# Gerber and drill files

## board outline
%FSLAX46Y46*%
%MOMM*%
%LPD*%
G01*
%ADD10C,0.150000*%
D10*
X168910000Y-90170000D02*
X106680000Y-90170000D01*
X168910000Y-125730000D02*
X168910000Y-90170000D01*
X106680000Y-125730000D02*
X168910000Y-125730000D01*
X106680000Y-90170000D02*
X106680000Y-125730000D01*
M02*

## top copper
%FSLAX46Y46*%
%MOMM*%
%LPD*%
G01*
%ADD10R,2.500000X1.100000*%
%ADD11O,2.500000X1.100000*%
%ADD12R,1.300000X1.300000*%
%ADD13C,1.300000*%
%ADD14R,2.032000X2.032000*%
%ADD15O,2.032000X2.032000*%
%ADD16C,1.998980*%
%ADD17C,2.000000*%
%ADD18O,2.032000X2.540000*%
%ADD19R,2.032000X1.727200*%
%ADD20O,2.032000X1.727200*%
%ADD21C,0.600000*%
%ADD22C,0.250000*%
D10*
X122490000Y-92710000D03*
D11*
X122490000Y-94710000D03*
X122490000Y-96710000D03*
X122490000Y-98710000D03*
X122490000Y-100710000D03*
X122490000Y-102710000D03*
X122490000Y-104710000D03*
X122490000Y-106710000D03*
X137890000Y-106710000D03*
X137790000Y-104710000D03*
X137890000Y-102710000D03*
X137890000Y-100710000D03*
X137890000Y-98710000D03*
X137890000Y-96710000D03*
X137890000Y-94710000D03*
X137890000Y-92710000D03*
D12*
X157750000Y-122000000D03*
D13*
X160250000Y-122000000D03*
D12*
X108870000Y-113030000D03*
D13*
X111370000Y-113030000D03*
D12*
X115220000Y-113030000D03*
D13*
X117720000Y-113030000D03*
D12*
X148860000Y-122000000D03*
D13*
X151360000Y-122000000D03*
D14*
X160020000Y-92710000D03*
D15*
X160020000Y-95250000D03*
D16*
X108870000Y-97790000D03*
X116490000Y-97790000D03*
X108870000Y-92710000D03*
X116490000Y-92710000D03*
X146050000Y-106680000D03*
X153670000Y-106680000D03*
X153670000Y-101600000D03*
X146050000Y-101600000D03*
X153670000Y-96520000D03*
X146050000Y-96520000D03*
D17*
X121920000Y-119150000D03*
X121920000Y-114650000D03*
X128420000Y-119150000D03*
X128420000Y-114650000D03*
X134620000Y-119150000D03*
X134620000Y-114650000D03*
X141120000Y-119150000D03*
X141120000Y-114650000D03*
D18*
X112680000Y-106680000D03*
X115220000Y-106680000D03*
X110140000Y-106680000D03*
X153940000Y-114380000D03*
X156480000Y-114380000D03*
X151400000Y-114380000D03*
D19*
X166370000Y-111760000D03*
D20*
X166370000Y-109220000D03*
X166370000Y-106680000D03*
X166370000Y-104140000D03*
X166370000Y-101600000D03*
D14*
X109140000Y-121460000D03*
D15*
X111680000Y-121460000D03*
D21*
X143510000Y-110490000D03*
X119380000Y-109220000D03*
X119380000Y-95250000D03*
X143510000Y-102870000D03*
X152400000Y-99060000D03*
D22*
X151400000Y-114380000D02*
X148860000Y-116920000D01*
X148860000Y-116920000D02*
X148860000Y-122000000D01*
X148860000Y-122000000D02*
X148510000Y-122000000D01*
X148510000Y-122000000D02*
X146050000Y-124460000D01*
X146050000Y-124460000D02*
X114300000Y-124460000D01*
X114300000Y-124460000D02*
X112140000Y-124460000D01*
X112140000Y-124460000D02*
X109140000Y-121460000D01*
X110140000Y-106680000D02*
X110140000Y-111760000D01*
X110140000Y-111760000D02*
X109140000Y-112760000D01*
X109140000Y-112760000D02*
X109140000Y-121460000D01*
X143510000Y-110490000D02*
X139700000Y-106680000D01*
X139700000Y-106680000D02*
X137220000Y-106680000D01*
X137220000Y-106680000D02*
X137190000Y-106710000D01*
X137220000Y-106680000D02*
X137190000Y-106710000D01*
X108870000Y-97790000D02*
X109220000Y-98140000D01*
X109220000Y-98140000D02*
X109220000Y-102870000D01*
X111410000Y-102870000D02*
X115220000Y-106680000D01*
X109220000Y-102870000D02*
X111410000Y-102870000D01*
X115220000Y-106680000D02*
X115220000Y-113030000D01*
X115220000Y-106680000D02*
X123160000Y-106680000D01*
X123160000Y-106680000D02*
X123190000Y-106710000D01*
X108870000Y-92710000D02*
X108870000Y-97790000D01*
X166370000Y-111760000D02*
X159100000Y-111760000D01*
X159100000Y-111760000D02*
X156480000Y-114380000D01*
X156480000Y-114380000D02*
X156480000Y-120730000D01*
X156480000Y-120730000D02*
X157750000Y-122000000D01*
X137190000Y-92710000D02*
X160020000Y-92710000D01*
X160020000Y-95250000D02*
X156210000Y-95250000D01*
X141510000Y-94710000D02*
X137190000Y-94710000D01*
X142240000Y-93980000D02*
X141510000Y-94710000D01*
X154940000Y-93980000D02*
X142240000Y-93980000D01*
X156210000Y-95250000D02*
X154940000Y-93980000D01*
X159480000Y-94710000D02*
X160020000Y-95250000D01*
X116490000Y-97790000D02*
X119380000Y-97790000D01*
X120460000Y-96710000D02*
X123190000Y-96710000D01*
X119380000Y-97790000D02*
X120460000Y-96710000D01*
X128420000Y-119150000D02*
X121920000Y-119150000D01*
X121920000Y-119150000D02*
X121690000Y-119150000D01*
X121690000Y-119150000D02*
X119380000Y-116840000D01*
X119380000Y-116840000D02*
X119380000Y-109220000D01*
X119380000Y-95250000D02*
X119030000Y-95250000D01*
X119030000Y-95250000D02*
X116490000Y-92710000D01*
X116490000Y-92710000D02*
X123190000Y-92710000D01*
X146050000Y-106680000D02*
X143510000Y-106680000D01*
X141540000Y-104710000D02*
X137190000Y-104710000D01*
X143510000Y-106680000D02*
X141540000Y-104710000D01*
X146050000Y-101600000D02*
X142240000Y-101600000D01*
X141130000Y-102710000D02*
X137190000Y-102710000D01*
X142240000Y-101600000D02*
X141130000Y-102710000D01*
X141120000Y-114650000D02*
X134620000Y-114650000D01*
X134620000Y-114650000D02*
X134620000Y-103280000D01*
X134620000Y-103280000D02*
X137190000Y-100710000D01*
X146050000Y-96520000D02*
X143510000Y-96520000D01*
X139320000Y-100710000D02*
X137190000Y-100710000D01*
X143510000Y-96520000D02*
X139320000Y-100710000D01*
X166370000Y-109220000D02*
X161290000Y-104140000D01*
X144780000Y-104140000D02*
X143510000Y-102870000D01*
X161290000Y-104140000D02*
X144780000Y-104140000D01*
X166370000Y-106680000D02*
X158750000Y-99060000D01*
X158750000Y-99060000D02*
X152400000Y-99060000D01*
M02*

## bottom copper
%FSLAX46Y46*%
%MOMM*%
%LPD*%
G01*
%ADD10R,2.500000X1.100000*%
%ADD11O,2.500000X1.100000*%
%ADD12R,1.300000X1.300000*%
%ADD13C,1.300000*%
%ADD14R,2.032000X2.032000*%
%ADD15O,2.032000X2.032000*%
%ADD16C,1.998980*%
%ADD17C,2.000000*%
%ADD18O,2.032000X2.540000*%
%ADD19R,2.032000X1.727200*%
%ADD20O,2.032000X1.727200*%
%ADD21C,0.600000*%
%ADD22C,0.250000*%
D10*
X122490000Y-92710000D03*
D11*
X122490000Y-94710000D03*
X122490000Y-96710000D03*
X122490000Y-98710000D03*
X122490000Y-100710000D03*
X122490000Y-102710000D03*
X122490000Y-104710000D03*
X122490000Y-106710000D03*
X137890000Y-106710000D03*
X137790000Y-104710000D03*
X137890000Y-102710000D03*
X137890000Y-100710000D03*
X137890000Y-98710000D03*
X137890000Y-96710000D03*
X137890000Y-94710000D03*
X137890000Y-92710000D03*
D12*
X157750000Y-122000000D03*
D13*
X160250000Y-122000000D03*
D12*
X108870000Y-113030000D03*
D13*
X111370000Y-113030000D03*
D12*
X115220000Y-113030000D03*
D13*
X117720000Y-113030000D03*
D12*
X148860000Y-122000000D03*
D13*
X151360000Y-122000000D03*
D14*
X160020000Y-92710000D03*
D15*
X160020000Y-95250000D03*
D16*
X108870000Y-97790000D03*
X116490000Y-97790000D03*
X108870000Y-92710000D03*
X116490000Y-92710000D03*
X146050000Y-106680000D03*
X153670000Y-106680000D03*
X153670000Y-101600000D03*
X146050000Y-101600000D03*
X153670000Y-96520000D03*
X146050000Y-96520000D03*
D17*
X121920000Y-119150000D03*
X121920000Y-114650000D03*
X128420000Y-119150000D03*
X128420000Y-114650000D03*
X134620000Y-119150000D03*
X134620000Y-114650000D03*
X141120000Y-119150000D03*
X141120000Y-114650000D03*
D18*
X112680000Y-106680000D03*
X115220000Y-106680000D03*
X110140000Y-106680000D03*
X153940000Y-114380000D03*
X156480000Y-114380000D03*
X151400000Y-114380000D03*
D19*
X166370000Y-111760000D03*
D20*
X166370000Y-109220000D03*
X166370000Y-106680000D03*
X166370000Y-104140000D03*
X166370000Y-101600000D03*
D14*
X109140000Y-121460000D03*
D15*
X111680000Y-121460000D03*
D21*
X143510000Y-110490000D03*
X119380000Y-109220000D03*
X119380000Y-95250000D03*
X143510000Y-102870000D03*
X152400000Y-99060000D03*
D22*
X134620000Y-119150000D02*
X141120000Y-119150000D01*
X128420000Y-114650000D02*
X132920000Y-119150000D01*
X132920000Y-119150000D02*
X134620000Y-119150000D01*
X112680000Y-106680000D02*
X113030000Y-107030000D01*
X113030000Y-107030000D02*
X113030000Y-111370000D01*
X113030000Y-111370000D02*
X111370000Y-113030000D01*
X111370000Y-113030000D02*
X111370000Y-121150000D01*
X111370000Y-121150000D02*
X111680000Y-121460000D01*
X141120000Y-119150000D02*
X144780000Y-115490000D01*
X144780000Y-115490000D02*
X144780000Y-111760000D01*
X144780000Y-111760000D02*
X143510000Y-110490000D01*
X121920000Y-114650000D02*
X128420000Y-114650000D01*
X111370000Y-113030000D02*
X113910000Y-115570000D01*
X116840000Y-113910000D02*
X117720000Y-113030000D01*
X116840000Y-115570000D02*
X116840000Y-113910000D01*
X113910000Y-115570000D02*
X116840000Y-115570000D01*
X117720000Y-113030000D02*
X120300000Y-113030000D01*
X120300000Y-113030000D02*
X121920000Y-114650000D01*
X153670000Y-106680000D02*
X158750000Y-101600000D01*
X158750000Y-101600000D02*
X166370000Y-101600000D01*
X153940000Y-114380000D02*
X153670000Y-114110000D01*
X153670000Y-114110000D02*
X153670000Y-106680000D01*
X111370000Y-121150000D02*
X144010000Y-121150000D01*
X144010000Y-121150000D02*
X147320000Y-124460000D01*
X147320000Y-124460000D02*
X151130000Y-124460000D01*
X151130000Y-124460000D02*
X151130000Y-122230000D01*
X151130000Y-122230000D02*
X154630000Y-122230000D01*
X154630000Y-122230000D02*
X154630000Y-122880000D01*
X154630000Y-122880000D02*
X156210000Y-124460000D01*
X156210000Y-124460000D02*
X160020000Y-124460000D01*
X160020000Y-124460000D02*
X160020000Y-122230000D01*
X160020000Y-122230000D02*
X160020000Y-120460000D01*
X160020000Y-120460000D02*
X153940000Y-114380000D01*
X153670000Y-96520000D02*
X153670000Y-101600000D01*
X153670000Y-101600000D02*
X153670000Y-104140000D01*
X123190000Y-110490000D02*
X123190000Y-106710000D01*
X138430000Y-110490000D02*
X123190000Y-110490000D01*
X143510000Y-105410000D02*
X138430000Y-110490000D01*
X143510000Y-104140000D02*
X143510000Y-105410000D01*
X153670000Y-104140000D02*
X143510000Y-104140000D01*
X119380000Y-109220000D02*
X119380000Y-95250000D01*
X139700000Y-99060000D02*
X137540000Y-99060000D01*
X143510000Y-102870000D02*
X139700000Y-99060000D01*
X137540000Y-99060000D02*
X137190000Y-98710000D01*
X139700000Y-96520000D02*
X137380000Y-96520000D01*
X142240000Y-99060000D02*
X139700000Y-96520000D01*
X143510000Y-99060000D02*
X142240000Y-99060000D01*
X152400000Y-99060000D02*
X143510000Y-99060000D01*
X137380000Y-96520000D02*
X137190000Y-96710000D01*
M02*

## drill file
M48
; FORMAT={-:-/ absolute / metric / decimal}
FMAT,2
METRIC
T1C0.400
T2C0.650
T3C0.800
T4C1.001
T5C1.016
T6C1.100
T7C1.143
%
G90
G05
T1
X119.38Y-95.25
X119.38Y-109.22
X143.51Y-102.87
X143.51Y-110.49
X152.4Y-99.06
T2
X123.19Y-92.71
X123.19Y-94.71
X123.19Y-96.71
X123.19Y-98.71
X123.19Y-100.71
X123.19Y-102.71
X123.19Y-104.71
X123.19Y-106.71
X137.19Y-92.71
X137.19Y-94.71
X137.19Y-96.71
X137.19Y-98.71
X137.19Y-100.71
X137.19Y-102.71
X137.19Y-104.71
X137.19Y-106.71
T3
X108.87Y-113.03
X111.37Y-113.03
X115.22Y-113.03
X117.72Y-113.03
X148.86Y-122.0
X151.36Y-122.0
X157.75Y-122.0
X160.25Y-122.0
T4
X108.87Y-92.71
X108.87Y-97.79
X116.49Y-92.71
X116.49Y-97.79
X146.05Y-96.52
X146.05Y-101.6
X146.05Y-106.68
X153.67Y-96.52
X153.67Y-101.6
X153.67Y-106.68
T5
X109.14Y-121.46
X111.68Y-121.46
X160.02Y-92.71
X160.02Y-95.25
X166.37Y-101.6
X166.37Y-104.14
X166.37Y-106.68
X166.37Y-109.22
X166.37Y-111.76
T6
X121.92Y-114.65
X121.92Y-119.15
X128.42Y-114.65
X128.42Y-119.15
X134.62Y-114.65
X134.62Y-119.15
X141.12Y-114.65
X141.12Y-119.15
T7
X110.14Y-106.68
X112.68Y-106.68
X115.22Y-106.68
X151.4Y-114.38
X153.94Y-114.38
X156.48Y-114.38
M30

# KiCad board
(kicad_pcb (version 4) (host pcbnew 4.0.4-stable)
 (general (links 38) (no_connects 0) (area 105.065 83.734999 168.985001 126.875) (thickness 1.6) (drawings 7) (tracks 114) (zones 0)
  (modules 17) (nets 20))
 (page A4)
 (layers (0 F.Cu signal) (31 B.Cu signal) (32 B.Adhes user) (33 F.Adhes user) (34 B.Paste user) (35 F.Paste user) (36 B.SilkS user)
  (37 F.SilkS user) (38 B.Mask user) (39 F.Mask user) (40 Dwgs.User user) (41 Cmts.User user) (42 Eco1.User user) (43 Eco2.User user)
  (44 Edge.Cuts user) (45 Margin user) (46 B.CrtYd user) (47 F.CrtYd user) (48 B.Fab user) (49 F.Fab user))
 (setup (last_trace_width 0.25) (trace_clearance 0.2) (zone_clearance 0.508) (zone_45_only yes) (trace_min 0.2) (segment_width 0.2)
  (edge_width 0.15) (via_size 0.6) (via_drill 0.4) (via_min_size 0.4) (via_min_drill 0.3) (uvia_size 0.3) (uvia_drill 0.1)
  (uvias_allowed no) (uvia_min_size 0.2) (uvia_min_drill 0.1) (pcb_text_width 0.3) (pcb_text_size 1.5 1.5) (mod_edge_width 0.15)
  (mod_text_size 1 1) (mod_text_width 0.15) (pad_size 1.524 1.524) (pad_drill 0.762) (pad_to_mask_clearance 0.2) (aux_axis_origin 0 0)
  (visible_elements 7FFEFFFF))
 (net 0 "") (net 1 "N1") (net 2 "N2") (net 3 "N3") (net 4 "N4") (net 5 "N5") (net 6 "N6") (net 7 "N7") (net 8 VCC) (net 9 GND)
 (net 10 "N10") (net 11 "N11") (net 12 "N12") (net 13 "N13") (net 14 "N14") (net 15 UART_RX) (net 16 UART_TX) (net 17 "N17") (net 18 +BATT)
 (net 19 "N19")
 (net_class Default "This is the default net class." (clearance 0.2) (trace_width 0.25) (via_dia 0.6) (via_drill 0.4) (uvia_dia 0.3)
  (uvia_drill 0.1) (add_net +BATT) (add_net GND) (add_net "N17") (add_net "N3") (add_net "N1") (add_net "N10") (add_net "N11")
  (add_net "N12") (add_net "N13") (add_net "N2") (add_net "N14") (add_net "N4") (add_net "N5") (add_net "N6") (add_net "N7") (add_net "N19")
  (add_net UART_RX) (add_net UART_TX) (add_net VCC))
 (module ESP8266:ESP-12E (layer F.Cu) (at 123.19 92.71)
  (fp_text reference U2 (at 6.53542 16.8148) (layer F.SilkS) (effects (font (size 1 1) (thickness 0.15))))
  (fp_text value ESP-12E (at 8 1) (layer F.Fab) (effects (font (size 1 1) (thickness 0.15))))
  (pad 1 thru_hole rect (at 0 0) (size 2.5 1.1) (drill 0.65 (offset -0.7 0)) (layers *.Cu *.Mask F.SilkS) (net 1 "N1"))
  (pad 2 thru_hole oval (at 0 2) (size 2.5 1.1) (drill 0.65 (offset -0.7 0)) (layers *.Cu *.Mask F.SilkS) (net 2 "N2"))
  (pad 3 thru_hole oval (at 0 4) (size 2.5 1.1) (drill 0.65 (offset -0.7 0)) (layers *.Cu *.Mask F.SilkS) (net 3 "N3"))
  (pad 4 thru_hole oval (at 0 6) (size 2.5 1.1) (drill 0.65 (offset -0.7 0)) (layers *.Cu *.Mask F.SilkS) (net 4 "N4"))
  (pad 5 thru_hole oval (at 0 8) (size 2.5 1.1) (drill 0.65 (offset -0.7 0)) (layers *.Cu *.Mask F.SilkS) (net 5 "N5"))
  (pad 6 thru_hole oval (at 0 10) (size 2.5 1.1) (drill 0.65 (offset -0.7 0)) (layers *.Cu *.Mask F.SilkS) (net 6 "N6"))
  (pad 7 thru_hole oval (at 0 12) (size 2.5 1.1) (drill 0.65 (offset -0.7 0)) (layers *.Cu *.Mask F.SilkS) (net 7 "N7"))
  (pad 8 thru_hole oval (at 0 14) (size 2.5 1.1) (drill 0.65 (offset -0.7 0)) (layers *.Cu *.Mask F.SilkS) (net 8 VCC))
  (pad 15 thru_hole oval (at 14 14) (size 2.5 1.1) (drill 0.65 (offset 0.7 0)) (layers *.Cu *.Mask F.SilkS) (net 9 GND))
  (pad 16 thru_hole oval (at 14 12) (size 2.5 1.1) (drill 0.65 (offset 0.6 0)) (layers *.Cu *.Mask F.SilkS) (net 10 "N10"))
  (pad 17 thru_hole oval (at 14 10) (size 2.5 1.1) (drill 0.65 (offset 0.7 0)) (layers *.Cu *.Mask F.SilkS) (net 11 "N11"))
  (pad 18 thru_hole oval (at 14 8) (size 2.5 1.1) (drill 0.65 (offset 0.7 0)) (layers *.Cu *.Mask F.SilkS) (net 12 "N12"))
  (pad 19 thru_hole oval (at 14 6) (size 2.5 1.1) (drill 0.65 (offset 0.7 0)) (layers *.Cu *.Mask F.SilkS) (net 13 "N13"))
  (pad 20 thru_hole oval (at 14 4) (size 2.5 1.1) (drill 0.65 (offset 0.7 0)) (layers *.Cu *.Mask F.SilkS) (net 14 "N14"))
  (pad 21 thru_hole oval (at 14 2) (size 2.5 1.1) (drill 0.65 (offset 0.7 0)) (layers *.Cu *.Mask F.SilkS) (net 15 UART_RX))
  (pad 22 thru_hole oval (at 14 0) (size 2.5 1.1) (drill 0.65 (offset 0.7 0)) (layers *.Cu *.Mask F.SilkS) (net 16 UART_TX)))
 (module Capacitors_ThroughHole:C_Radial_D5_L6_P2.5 (layer F.Cu) (at 157.75 122)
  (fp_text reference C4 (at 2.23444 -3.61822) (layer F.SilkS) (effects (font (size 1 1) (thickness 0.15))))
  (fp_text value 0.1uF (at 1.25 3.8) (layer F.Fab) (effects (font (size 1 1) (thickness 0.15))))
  (pad 1 thru_hole rect (at 0 0) (size 1.3 1.3) (drill 0.8) (layers *.Cu *.Mask) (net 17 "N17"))
  (pad 2 thru_hole circle (at 2.5 0) (size 1.3 1.3) (drill 0.8) (layers *.Cu *.Mask) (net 9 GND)))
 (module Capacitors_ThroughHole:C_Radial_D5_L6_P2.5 (layer F.Cu) (at 108.87 113.03)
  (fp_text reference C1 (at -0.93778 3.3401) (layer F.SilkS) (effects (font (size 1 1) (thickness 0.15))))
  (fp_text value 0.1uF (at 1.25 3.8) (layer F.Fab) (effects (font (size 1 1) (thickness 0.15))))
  (pad 1 thru_hole rect (at 0 0) (size 1.3 1.3) (drill 0.8) (layers *.Cu *.Mask) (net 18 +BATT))
  (pad 2 thru_hole circle (at 2.5 0) (size 1.3 1.3) (drill 0.8) (layers *.Cu *.Mask) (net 9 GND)))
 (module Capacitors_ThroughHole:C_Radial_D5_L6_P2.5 (layer F.Cu) (at 115.22 113.03)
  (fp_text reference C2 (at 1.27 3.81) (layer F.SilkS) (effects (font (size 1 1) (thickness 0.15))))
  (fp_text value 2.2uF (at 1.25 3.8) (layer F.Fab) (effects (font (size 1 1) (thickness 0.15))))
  (pad 1 thru_hole rect (at 0 0) (size 1.3 1.3) (drill 0.8) (layers *.Cu *.Mask) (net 8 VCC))
  (pad 2 thru_hole circle (at 2.5 0) (size 1.3 1.3) (drill 0.8) (layers *.Cu *.Mask) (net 9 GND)))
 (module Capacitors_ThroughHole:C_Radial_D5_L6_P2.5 (layer F.Cu) (at 148.86 122)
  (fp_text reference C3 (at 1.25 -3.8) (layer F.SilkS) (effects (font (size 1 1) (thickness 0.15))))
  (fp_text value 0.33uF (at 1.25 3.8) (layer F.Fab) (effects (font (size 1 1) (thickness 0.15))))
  (pad 1 thru_hole rect (at 0 0) (size 1.3 1.3) (drill 0.8) (layers *.Cu *.Mask) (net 18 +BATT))
  (pad 2 thru_hole circle (at 2.5 0) (size 1.3 1.3) (drill 0.8) (layers *.Cu *.Mask) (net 9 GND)))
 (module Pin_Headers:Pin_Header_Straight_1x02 (layer F.Cu) (at 160.02 92.71)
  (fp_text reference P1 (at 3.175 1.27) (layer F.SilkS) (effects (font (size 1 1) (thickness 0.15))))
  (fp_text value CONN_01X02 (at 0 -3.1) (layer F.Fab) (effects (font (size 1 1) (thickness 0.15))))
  (pad 1 thru_hole rect (at 0 0) (size 2.032 2.032) (drill 1.016) (layers *.Cu *.Mask) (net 16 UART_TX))
  (pad 2 thru_hole oval (at 0 2.54) (size 2.032 2.032) (drill 1.016) (layers *.Cu *.Mask) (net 15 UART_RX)))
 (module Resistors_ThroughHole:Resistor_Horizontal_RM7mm (layer F.Cu) (at 108.87 97.79)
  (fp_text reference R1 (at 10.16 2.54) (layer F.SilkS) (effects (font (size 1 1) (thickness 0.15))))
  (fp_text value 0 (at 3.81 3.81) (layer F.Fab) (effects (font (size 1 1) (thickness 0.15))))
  (pad 1 thru_hole circle (at 0 0) (size 1.99898 1.99898) (drill 1.00076) (layers *.Cu *.SilkS *.Mask) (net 8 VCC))
  (pad 2 thru_hole circle (at 7.62 0) (size 1.99898 1.99898) (drill 1.00076) (layers *.Cu *.SilkS *.Mask) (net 3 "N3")))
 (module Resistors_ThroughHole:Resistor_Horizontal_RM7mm (layer F.Cu) (at 108.87 92.71)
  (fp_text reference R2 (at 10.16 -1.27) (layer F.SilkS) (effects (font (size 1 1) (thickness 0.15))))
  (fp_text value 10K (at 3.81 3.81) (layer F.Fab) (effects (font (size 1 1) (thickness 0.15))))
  (pad 1 thru_hole circle (at 0 0) (size 1.99898 1.99898) (drill 1.00076) (layers *.Cu *.SilkS *.Mask) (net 8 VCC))
  (pad 2 thru_hole circle (at 7.62 0) (size 1.99898 1.99898) (drill 1.00076) (layers *.Cu *.SilkS *.Mask) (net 1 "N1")))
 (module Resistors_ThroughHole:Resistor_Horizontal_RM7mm (layer F.Cu) (at 146.05 106.68)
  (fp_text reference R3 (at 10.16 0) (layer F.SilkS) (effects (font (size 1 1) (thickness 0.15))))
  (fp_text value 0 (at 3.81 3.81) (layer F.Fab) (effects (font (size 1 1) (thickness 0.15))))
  (pad 1 thru_hole circle (at 0 0) (size 1.99898 1.99898) (drill 1.00076) (layers *.Cu *.SilkS *.Mask) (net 10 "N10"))
  (pad 2 thru_hole circle (at 7.62 0) (size 1.99898 1.99898) (drill 1.00076) (layers *.Cu *.SilkS *.Mask) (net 9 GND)))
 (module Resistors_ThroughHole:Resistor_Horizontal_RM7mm (layer F.Cu) (at 153.67 101.6 180)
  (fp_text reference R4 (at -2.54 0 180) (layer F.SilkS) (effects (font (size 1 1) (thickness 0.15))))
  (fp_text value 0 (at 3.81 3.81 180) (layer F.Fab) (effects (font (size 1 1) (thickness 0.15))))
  (pad 1 thru_hole circle (at 0 0 180) (size 1.99898 1.99898) (drill 1.00076) (layers *.Cu *.SilkS *.Mask) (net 8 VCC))
  (pad 2 thru_hole circle (at 7.62 0 180) (size 1.99898 1.99898) (drill 1.00076) (layers *.Cu *.SilkS *.Mask) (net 11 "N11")))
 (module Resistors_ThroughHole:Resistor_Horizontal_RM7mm (layer F.Cu) (at 153.67 96.52 180)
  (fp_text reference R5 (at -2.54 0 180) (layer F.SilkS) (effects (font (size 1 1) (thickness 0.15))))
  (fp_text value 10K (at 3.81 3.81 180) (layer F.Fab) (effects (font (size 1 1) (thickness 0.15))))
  (pad 1 thru_hole circle (at 0 0 180) (size 1.99898 1.99898) (drill 1.00076) (layers *.Cu *.SilkS *.Mask) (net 8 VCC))
  (pad 2 thru_hole circle (at 7.62 0 180) (size 1.99898 1.99898) (drill 1.00076) (layers *.Cu *.SilkS *.Mask) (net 12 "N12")))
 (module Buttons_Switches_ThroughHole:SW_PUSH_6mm (layer F.Cu) (at 121.92 114.65)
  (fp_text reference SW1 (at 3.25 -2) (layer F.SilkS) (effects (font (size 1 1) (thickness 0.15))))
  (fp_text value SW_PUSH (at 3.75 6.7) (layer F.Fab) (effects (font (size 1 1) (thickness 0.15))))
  (pad 2 thru_hole circle (at 0 4.5 90) (size 2 2) (drill 1.1) (layers *.Cu *.Mask) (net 1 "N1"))
  (pad 1 thru_hole circle (at 0 0 90) (size 2 2) (drill 1.1) (layers *.Cu *.Mask) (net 9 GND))
  (pad 2 thru_hole circle (at 6.5 4.5 90) (size 2 2) (drill 1.1) (layers *.Cu *.Mask) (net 1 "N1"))
  (pad 1 thru_hole circle (at 6.5 0 90) (size 2 2) (drill 1.1) (layers *.Cu *.Mask) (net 9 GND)))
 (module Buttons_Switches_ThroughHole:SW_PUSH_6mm (layer F.Cu) (at 134.62 114.65)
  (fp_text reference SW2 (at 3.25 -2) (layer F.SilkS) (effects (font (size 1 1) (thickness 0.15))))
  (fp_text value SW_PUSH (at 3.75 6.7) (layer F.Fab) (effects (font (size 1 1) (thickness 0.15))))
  (pad 2 thru_hole circle (at 0 4.5 90) (size 2 2) (drill 1.1) (layers *.Cu *.Mask) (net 9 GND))
  (pad 1 thru_hole circle (at 0 0 90) (size 2 2) (drill 1.1) (layers *.Cu *.Mask) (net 12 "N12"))
  (pad 2 thru_hole circle (at 6.5 4.5 90) (size 2 2) (drill 1.1) (layers *.Cu *.Mask) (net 9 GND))
  (pad 1 thru_hole circle (at 6.5 0 90) (size 2 2) (drill 1.1) (layers *.Cu *.Mask) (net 12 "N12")))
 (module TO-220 (layer F.Cu) (at 112.68 106.68)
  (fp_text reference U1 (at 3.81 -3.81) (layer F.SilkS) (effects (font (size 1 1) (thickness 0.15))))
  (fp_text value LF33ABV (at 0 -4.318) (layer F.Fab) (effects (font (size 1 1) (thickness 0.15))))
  (pad 2 thru_hole oval (at 0 0) (size 2.032 2.54) (drill 1.143) (layers *.Cu *.Mask) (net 9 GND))
  (pad 3 thru_hole oval (at 2.54 0) (size 2.032 2.54) (drill 1.143) (layers *.Cu *.Mask) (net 8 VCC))
  (pad 1 thru_hole oval (at -2.54 0) (size 2.032 2.54) (drill 1.143) (layers *.Cu *.Mask) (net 18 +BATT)))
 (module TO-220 (layer F.Cu) (at 153.94 114.38)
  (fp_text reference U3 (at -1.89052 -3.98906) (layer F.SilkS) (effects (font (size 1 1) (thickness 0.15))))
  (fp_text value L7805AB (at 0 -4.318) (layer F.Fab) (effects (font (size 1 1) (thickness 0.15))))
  (pad 2 thru_hole oval (at 0 0) (size 2.032 2.54) (drill 1.143) (layers *.Cu *.Mask) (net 9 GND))
  (pad 3 thru_hole oval (at 2.54 0) (size 2.032 2.54) (drill 1.143) (layers *.Cu *.Mask) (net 17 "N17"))
  (pad 1 thru_hole oval (at -2.54 0) (size 2.032 2.54) (drill 1.143) (layers *.Cu *.Mask) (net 18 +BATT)))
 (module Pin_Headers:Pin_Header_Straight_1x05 (layer F.Cu) (at 166.37 111.76 180)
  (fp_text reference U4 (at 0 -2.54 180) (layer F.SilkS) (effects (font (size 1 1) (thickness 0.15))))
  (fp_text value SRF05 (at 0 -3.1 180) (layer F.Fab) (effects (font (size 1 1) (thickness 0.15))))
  (pad 1 thru_hole rect (at 0 0 180) (size 2.032 1.7272) (drill 1.016) (layers *.Cu *.Mask) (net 17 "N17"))
  (pad 2 thru_hole oval (at 0 2.54 180) (size 2.032 1.7272) (drill 1.016) (layers *.Cu *.Mask) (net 13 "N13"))
  (pad 3 thru_hole oval (at 0 5.08 180) (size 2.032 1.7272) (drill 1.016) (layers *.Cu *.Mask) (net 14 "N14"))
  (pad 4 thru_hole oval (at 0 7.62 180) (size 2.032 1.7272) (drill 1.016) (layers *.Cu *.Mask) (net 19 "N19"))
  (pad 5 thru_hole oval (at 0 10.16 180) (size 2.032 1.7272) (drill 1.016) (layers *.Cu *.Mask) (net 9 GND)))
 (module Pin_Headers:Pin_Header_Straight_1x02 (layer F.Cu) (at 109.14 121.46 90)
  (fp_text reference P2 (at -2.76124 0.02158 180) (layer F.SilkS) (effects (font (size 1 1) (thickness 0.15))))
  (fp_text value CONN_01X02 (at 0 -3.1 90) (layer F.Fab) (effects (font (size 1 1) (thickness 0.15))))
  (pad 1 thru_hole rect (at 0 0 90) (size 2.032 2.032) (drill 1.016) (layers *.Cu *.Mask) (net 18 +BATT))
  (pad 2 thru_hole oval (at 0 2.54 90) (size 2.032 2.032) (drill 1.016) (layers *.Cu *.Mask) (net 9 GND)))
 (gr_line (start 168.91 90.17) (end 106.68 90.17) (angle 90) (layer Edge.Cuts) (width 0.15))
 (gr_line (start 168.91 125.73) (end 168.91 90.17) (angle 90) (layer Edge.Cuts) (width 0.15))
 (gr_line (start 106.68 125.73) (end 168.91 125.73) (angle 90) (layer Edge.Cuts) (width 0.15))
 (gr_line (start 106.68 90.17) (end 106.68 125.73) (angle 90) (layer Edge.Cuts) (width 0.15))
 (segment (start 151.4 114.38) (end 148.86 116.92) (width 0.25) (layer F.Cu) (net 18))
 (segment (start 148.86 116.92) (end 148.86 122) (width 0.25) (layer F.Cu) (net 18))
 (segment (start 148.86 122) (end 148.51 122) (width 0.25) (layer F.Cu) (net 18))
 (segment (start 148.51 122) (end 146.05 124.46) (width 0.25) (layer F.Cu) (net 18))
 (segment (start 146.05 124.46) (end 114.3 124.46) (width 0.25) (layer F.Cu) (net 18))
 (segment (start 114.3 124.46) (end 112.14 124.46) (width 0.25) (layer F.Cu) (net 18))
 (segment (start 112.14 124.46) (end 109.14 121.46) (width 0.25) (layer F.Cu) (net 18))
 (segment (start 110.14 106.68) (end 110.14 111.76) (width 0.25) (layer F.Cu) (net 18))
 (segment (start 110.14 111.76) (end 109.14 112.76) (width 0.25) (layer F.Cu) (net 18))
 (segment (start 109.14 112.76) (end 109.14 121.46) (width 0.25) (layer F.Cu) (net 18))
 (segment (start 134.62 119.15) (end 141.12 119.15) (width 0.25) (layer B.Cu) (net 9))
 (segment (start 128.42 114.65) (end 132.92 119.15) (width 0.25) (layer B.Cu) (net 9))
 (segment (start 132.92 119.15) (end 134.62 119.15) (width 0.25) (layer B.Cu) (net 9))
 (segment (start 112.68 106.68) (end 113.03 107.03) (width 0.25) (layer B.Cu) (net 9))
 (segment (start 113.03 107.03) (end 113.03 111.37) (width 0.25) (layer B.Cu) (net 9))
 (segment (start 113.03 111.37) (end 111.37 113.03) (width 0.25) (layer B.Cu) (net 9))
 (segment (start 111.37 113.03) (end 111.37 121.15) (width 0.25) (layer B.Cu) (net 9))
 (segment (start 111.37 121.15) (end 111.68 121.46) (width 0.25) (layer B.Cu) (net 9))
 (segment (start 141.12 119.15) (end 144.78 115.49) (width 0.25) (layer B.Cu) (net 9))
 (segment (start 144.78 115.49) (end 144.78 111.76) (width 0.25) (layer B.Cu) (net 9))
 (segment (start 144.78 111.76) (end 143.51 110.49) (width 0.25) (layer B.Cu) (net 9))
 (via (at 143.51 110.49) (size 0.6) (drill 0.4) (layers F.Cu B.Cu) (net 9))
 (segment (start 143.51 110.49) (end 139.7 106.68) (width 0.25) (layer F.Cu) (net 9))
 (segment (start 139.7 106.68) (end 137.22 106.68) (width 0.25) (layer F.Cu) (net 9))
 (segment (start 137.22 106.68) (end 137.19 106.71) (width 0.25) (layer F.Cu) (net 9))
 (segment (start 137.22 106.68) (end 137.19 106.71) (width 0.25) (layer F.Cu) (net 9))
 (segment (start 121.92 114.65) (end 128.42 114.65) (width 0.25) (layer B.Cu) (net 9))
 (segment (start 111.37 113.03) (end 113.91 115.57) (width 0.25) (layer B.Cu) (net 9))
 (segment (start 116.84 113.91) (end 117.72 113.03) (width 0.25) (layer B.Cu) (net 9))
 (segment (start 116.84 115.57) (end 116.84 113.91) (width 0.25) (layer B.Cu) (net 9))
 (segment (start 113.91 115.57) (end 116.84 115.57) (width 0.25) (layer B.Cu) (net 9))
 (segment (start 117.72 113.03) (end 120.3 113.03) (width 0.25) (layer B.Cu) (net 9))
 (segment (start 120.3 113.03) (end 121.92 114.65) (width 0.25) (layer B.Cu) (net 9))
 (segment (start 153.67 106.68) (end 158.75 101.6) (width 0.25) (layer B.Cu) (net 9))
 (segment (start 158.75 101.6) (end 166.37 101.6) (width 0.25) (layer B.Cu) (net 9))
 (segment (start 153.94 114.38) (end 153.67 114.11) (width 0.25) (layer B.Cu) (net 9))
 (segment (start 153.67 114.11) (end 153.67 106.68) (width 0.25) (layer B.Cu) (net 9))
 (segment (start 111.37 121.15) (end 144.01 121.15) (width 0.25) (layer B.Cu) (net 9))
 (segment (start 144.01 121.15) (end 147.32 124.46) (width 0.25) (layer B.Cu) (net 9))
 (segment (start 147.32 124.46) (end 151.13 124.46) (width 0.25) (layer B.Cu) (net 9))
 (segment (start 151.13 124.46) (end 151.13 122.23) (width 0.25) (layer B.Cu) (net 9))
 (segment (start 151.13 122.23) (end 154.63 122.23) (width 0.25) (layer B.Cu) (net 9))
 (segment (start 154.63 122.23) (end 154.63 122.88) (width 0.25) (layer B.Cu) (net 9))
 (segment (start 154.63 122.88) (end 156.21 124.46) (width 0.25) (layer B.Cu) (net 9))
 (segment (start 156.21 124.46) (end 160.02 124.46) (width 0.25) (layer B.Cu) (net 9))
 (segment (start 160.02 124.46) (end 160.02 122.23) (width 0.25) (layer B.Cu) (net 9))
 (segment (start 160.02 122.23) (end 160.02 120.46) (width 0.25) (layer B.Cu) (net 9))
 (segment (start 160.02 120.46) (end 153.94 114.38) (width 0.25) (layer B.Cu) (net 9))
 (segment (start 108.87 97.79) (end 109.22 98.14) (width 0.25) (layer F.Cu) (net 8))
 (segment (start 109.22 98.14) (end 109.22 102.87) (width 0.25) (layer F.Cu) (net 8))
 (segment (start 111.41 102.87) (end 115.22 106.68) (width 0.25) (layer F.Cu) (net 8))
 (segment (start 109.22 102.87) (end 111.41 102.87) (width 0.25) (layer F.Cu) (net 8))
 (segment (start 115.22 106.68) (end 115.22 113.03) (width 0.25) (layer F.Cu) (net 8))
 (segment (start 153.67 96.52) (end 153.67 101.6) (width 0.25) (layer B.Cu) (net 8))
 (segment (start 153.67 101.6) (end 153.67 104.14) (width 0.25) (layer B.Cu) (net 8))
 (segment (start 123.19 110.49) (end 123.19 106.71) (width 0.25) (layer B.Cu) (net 8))
 (segment (start 138.43 110.49) (end 123.19 110.49) (width 0.25) (layer B.Cu) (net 8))
 (segment (start 143.51 105.41) (end 138.43 110.49) (width 0.25) (layer B.Cu) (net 8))
 (segment (start 143.51 104.14) (end 143.51 105.41) (width 0.25) (layer B.Cu) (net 8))
 (segment (start 153.67 104.14) (end 143.51 104.14) (width 0.25) (layer B.Cu) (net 8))
 (segment (start 115.22 106.68) (end 123.16 106.68) (width 0.25) (layer F.Cu) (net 8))
 (segment (start 123.16 106.68) (end 123.19 106.71) (width 0.25) (layer F.Cu) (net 8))
 (segment (start 108.87 92.71) (end 108.87 97.79) (width 0.25) (layer F.Cu) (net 8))
 (segment (start 166.37 111.76) (end 159.1 111.76) (width 0.25) (layer F.Cu) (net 17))
 (segment (start 159.1 111.76) (end 156.48 114.38) (width 0.25) (layer F.Cu) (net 17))
 (segment (start 156.48 114.38) (end 156.48 120.73) (width 0.25) (layer F.Cu) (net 17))
 (segment (start 156.48 120.73) (end 157.75 122) (width 0.25) (layer F.Cu) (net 17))
 (segment (start 137.19 92.71) (end 160.02 92.71) (width 0.25) (layer F.Cu) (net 16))
 (segment (start 160.02 95.25) (end 156.21 95.25) (width 0.25) (layer F.Cu) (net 15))
 (segment (start 141.51 94.71) (end 137.19 94.71) (width 0.25) (layer F.Cu) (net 15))
 (segment (start 142.24 93.98) (end 141.51 94.71) (width 0.25) (layer F.Cu) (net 15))
 (segment (start 154.94 93.98) (end 142.24 93.98) (width 0.25) (layer F.Cu) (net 15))
 (segment (start 156.21 95.25) (end 154.94 93.98) (width 0.25) (layer F.Cu) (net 15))
 (segment (start 159.48 94.71) (end 160.02 95.25) (width 0.25) (layer F.Cu) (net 15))
 (segment (start 116.49 97.79) (end 119.38 97.79) (width 0.25) (layer F.Cu) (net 3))
 (segment (start 120.46 96.71) (end 123.19 96.71) (width 0.25) (layer F.Cu) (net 3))
 (segment (start 119.38 97.79) (end 120.46 96.71) (width 0.25) (layer F.Cu) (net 3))
 (segment (start 128.42 119.15) (end 121.92 119.15) (width 0.25) (layer F.Cu) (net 1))
 (segment (start 121.92 119.15) (end 121.69 119.15) (width 0.25) (layer F.Cu) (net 1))
 (segment (start 121.69 119.15) (end 119.38 116.84) (width 0.25) (layer F.Cu) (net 1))
 (segment (start 119.38 116.84) (end 119.38 109.22) (width 0.25) (layer F.Cu) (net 1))
 (via (at 119.38 109.22) (size 0.6) (drill 0.4) (layers F.Cu B.Cu) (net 1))
 (segment (start 119.38 109.22) (end 119.38 95.25) (width 0.25) (layer B.Cu) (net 1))
 (via (at 119.38 95.25) (size 0.6) (drill 0.4) (layers F.Cu B.Cu) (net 1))
 (segment (start 119.38 95.25) (end 119.03 95.25) (width 0.25) (layer F.Cu) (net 1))
 (segment (start 119.03 95.25) (end 116.49 92.71) (width 0.25) (layer F.Cu) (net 1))
 (segment (start 116.49 92.71) (end 123.19 92.71) (width 0.25) (layer F.Cu) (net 1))
 (segment (start 146.05 106.68) (end 143.51 106.68) (width 0.25) (layer F.Cu) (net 10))
 (segment (start 141.54 104.71) (end 137.19 104.71) (width 0.25) (layer F.Cu) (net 10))
 (segment (start 143.51 106.68) (end 141.54 104.71) (width 0.25) (layer F.Cu) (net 10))
 (segment (start 146.05 101.6) (end 142.24 101.6) (width 0.25) (layer F.Cu) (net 11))
 (segment (start 141.13 102.71) (end 137.19 102.71) (width 0.25) (layer F.Cu) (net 11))
 (segment (start 142.24 101.6) (end 141.13 102.71) (width 0.25) (layer F.Cu) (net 11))
 (segment (start 141.12 114.65) (end 134.62 114.65) (width 0.25) (layer F.Cu) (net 12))
 (segment (start 134.62 114.65) (end 134.62 103.28) (width 0.25) (layer F.Cu) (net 12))
 (segment (start 134.62 103.28) (end 137.19 100.71) (width 0.25) (layer F.Cu) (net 12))
 (segment (start 146.05 96.52) (end 143.51 96.52) (width 0.25) (layer F.Cu) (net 12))
 (segment (start 139.32 100.71) (end 137.19 100.71) (width 0.25) (layer F.Cu) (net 12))
 (segment (start 143.51 96.52) (end 139.32 100.71) (width 0.25) (layer F.Cu) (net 12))
 (segment (start 166.37 109.22) (end 161.29 104.14) (width 0.25) (layer F.Cu) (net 13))
 (segment (start 139.7 99.06) (end 137.54 99.06) (width 0.25) (layer B.Cu) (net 13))
 (segment (start 143.51 102.87) (end 139.7 99.06) (width 0.25) (layer B.Cu) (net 13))
 (via (at 143.51 102.87) (size 0.6) (drill 0.4) (layers F.Cu B.Cu) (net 13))
 (segment (start 144.78 104.14) (end 143.51 102.87) (width 0.25) (layer F.Cu) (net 13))
 (segment (start 161.29 104.14) (end 144.78 104.14) (width 0.25) (layer F.Cu) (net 13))
 (segment (start 137.54 99.06) (end 137.19 98.71) (width 0.25) (layer B.Cu) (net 13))
 (segment (start 166.37 106.68) (end 158.75 99.06) (width 0.25) (layer F.Cu) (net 14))
 (segment (start 139.7 96.52) (end 137.38 96.52) (width 0.25) (layer B.Cu) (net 14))
 (segment (start 142.24 99.06) (end 139.7 96.52) (width 0.25) (layer B.Cu) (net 14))
 (segment (start 143.51 99.06) (end 142.24 99.06) (width 0.25) (layer B.Cu) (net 14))
 (segment (start 152.4 99.06) (end 143.51 99.06) (width 0.25) (layer B.Cu) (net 14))
 (via (at 152.4 99.06) (size 0.6) (drill 0.4) (layers F.Cu B.Cu) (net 14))
 (segment (start 158.75 99.06) (end 152.4 99.06) (width 0.25) (layer F.Cu) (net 14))
 (segment (start 137.38 96.52) (end 137.19 96.71) (width 0.25) (layer B.Cu) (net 14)))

